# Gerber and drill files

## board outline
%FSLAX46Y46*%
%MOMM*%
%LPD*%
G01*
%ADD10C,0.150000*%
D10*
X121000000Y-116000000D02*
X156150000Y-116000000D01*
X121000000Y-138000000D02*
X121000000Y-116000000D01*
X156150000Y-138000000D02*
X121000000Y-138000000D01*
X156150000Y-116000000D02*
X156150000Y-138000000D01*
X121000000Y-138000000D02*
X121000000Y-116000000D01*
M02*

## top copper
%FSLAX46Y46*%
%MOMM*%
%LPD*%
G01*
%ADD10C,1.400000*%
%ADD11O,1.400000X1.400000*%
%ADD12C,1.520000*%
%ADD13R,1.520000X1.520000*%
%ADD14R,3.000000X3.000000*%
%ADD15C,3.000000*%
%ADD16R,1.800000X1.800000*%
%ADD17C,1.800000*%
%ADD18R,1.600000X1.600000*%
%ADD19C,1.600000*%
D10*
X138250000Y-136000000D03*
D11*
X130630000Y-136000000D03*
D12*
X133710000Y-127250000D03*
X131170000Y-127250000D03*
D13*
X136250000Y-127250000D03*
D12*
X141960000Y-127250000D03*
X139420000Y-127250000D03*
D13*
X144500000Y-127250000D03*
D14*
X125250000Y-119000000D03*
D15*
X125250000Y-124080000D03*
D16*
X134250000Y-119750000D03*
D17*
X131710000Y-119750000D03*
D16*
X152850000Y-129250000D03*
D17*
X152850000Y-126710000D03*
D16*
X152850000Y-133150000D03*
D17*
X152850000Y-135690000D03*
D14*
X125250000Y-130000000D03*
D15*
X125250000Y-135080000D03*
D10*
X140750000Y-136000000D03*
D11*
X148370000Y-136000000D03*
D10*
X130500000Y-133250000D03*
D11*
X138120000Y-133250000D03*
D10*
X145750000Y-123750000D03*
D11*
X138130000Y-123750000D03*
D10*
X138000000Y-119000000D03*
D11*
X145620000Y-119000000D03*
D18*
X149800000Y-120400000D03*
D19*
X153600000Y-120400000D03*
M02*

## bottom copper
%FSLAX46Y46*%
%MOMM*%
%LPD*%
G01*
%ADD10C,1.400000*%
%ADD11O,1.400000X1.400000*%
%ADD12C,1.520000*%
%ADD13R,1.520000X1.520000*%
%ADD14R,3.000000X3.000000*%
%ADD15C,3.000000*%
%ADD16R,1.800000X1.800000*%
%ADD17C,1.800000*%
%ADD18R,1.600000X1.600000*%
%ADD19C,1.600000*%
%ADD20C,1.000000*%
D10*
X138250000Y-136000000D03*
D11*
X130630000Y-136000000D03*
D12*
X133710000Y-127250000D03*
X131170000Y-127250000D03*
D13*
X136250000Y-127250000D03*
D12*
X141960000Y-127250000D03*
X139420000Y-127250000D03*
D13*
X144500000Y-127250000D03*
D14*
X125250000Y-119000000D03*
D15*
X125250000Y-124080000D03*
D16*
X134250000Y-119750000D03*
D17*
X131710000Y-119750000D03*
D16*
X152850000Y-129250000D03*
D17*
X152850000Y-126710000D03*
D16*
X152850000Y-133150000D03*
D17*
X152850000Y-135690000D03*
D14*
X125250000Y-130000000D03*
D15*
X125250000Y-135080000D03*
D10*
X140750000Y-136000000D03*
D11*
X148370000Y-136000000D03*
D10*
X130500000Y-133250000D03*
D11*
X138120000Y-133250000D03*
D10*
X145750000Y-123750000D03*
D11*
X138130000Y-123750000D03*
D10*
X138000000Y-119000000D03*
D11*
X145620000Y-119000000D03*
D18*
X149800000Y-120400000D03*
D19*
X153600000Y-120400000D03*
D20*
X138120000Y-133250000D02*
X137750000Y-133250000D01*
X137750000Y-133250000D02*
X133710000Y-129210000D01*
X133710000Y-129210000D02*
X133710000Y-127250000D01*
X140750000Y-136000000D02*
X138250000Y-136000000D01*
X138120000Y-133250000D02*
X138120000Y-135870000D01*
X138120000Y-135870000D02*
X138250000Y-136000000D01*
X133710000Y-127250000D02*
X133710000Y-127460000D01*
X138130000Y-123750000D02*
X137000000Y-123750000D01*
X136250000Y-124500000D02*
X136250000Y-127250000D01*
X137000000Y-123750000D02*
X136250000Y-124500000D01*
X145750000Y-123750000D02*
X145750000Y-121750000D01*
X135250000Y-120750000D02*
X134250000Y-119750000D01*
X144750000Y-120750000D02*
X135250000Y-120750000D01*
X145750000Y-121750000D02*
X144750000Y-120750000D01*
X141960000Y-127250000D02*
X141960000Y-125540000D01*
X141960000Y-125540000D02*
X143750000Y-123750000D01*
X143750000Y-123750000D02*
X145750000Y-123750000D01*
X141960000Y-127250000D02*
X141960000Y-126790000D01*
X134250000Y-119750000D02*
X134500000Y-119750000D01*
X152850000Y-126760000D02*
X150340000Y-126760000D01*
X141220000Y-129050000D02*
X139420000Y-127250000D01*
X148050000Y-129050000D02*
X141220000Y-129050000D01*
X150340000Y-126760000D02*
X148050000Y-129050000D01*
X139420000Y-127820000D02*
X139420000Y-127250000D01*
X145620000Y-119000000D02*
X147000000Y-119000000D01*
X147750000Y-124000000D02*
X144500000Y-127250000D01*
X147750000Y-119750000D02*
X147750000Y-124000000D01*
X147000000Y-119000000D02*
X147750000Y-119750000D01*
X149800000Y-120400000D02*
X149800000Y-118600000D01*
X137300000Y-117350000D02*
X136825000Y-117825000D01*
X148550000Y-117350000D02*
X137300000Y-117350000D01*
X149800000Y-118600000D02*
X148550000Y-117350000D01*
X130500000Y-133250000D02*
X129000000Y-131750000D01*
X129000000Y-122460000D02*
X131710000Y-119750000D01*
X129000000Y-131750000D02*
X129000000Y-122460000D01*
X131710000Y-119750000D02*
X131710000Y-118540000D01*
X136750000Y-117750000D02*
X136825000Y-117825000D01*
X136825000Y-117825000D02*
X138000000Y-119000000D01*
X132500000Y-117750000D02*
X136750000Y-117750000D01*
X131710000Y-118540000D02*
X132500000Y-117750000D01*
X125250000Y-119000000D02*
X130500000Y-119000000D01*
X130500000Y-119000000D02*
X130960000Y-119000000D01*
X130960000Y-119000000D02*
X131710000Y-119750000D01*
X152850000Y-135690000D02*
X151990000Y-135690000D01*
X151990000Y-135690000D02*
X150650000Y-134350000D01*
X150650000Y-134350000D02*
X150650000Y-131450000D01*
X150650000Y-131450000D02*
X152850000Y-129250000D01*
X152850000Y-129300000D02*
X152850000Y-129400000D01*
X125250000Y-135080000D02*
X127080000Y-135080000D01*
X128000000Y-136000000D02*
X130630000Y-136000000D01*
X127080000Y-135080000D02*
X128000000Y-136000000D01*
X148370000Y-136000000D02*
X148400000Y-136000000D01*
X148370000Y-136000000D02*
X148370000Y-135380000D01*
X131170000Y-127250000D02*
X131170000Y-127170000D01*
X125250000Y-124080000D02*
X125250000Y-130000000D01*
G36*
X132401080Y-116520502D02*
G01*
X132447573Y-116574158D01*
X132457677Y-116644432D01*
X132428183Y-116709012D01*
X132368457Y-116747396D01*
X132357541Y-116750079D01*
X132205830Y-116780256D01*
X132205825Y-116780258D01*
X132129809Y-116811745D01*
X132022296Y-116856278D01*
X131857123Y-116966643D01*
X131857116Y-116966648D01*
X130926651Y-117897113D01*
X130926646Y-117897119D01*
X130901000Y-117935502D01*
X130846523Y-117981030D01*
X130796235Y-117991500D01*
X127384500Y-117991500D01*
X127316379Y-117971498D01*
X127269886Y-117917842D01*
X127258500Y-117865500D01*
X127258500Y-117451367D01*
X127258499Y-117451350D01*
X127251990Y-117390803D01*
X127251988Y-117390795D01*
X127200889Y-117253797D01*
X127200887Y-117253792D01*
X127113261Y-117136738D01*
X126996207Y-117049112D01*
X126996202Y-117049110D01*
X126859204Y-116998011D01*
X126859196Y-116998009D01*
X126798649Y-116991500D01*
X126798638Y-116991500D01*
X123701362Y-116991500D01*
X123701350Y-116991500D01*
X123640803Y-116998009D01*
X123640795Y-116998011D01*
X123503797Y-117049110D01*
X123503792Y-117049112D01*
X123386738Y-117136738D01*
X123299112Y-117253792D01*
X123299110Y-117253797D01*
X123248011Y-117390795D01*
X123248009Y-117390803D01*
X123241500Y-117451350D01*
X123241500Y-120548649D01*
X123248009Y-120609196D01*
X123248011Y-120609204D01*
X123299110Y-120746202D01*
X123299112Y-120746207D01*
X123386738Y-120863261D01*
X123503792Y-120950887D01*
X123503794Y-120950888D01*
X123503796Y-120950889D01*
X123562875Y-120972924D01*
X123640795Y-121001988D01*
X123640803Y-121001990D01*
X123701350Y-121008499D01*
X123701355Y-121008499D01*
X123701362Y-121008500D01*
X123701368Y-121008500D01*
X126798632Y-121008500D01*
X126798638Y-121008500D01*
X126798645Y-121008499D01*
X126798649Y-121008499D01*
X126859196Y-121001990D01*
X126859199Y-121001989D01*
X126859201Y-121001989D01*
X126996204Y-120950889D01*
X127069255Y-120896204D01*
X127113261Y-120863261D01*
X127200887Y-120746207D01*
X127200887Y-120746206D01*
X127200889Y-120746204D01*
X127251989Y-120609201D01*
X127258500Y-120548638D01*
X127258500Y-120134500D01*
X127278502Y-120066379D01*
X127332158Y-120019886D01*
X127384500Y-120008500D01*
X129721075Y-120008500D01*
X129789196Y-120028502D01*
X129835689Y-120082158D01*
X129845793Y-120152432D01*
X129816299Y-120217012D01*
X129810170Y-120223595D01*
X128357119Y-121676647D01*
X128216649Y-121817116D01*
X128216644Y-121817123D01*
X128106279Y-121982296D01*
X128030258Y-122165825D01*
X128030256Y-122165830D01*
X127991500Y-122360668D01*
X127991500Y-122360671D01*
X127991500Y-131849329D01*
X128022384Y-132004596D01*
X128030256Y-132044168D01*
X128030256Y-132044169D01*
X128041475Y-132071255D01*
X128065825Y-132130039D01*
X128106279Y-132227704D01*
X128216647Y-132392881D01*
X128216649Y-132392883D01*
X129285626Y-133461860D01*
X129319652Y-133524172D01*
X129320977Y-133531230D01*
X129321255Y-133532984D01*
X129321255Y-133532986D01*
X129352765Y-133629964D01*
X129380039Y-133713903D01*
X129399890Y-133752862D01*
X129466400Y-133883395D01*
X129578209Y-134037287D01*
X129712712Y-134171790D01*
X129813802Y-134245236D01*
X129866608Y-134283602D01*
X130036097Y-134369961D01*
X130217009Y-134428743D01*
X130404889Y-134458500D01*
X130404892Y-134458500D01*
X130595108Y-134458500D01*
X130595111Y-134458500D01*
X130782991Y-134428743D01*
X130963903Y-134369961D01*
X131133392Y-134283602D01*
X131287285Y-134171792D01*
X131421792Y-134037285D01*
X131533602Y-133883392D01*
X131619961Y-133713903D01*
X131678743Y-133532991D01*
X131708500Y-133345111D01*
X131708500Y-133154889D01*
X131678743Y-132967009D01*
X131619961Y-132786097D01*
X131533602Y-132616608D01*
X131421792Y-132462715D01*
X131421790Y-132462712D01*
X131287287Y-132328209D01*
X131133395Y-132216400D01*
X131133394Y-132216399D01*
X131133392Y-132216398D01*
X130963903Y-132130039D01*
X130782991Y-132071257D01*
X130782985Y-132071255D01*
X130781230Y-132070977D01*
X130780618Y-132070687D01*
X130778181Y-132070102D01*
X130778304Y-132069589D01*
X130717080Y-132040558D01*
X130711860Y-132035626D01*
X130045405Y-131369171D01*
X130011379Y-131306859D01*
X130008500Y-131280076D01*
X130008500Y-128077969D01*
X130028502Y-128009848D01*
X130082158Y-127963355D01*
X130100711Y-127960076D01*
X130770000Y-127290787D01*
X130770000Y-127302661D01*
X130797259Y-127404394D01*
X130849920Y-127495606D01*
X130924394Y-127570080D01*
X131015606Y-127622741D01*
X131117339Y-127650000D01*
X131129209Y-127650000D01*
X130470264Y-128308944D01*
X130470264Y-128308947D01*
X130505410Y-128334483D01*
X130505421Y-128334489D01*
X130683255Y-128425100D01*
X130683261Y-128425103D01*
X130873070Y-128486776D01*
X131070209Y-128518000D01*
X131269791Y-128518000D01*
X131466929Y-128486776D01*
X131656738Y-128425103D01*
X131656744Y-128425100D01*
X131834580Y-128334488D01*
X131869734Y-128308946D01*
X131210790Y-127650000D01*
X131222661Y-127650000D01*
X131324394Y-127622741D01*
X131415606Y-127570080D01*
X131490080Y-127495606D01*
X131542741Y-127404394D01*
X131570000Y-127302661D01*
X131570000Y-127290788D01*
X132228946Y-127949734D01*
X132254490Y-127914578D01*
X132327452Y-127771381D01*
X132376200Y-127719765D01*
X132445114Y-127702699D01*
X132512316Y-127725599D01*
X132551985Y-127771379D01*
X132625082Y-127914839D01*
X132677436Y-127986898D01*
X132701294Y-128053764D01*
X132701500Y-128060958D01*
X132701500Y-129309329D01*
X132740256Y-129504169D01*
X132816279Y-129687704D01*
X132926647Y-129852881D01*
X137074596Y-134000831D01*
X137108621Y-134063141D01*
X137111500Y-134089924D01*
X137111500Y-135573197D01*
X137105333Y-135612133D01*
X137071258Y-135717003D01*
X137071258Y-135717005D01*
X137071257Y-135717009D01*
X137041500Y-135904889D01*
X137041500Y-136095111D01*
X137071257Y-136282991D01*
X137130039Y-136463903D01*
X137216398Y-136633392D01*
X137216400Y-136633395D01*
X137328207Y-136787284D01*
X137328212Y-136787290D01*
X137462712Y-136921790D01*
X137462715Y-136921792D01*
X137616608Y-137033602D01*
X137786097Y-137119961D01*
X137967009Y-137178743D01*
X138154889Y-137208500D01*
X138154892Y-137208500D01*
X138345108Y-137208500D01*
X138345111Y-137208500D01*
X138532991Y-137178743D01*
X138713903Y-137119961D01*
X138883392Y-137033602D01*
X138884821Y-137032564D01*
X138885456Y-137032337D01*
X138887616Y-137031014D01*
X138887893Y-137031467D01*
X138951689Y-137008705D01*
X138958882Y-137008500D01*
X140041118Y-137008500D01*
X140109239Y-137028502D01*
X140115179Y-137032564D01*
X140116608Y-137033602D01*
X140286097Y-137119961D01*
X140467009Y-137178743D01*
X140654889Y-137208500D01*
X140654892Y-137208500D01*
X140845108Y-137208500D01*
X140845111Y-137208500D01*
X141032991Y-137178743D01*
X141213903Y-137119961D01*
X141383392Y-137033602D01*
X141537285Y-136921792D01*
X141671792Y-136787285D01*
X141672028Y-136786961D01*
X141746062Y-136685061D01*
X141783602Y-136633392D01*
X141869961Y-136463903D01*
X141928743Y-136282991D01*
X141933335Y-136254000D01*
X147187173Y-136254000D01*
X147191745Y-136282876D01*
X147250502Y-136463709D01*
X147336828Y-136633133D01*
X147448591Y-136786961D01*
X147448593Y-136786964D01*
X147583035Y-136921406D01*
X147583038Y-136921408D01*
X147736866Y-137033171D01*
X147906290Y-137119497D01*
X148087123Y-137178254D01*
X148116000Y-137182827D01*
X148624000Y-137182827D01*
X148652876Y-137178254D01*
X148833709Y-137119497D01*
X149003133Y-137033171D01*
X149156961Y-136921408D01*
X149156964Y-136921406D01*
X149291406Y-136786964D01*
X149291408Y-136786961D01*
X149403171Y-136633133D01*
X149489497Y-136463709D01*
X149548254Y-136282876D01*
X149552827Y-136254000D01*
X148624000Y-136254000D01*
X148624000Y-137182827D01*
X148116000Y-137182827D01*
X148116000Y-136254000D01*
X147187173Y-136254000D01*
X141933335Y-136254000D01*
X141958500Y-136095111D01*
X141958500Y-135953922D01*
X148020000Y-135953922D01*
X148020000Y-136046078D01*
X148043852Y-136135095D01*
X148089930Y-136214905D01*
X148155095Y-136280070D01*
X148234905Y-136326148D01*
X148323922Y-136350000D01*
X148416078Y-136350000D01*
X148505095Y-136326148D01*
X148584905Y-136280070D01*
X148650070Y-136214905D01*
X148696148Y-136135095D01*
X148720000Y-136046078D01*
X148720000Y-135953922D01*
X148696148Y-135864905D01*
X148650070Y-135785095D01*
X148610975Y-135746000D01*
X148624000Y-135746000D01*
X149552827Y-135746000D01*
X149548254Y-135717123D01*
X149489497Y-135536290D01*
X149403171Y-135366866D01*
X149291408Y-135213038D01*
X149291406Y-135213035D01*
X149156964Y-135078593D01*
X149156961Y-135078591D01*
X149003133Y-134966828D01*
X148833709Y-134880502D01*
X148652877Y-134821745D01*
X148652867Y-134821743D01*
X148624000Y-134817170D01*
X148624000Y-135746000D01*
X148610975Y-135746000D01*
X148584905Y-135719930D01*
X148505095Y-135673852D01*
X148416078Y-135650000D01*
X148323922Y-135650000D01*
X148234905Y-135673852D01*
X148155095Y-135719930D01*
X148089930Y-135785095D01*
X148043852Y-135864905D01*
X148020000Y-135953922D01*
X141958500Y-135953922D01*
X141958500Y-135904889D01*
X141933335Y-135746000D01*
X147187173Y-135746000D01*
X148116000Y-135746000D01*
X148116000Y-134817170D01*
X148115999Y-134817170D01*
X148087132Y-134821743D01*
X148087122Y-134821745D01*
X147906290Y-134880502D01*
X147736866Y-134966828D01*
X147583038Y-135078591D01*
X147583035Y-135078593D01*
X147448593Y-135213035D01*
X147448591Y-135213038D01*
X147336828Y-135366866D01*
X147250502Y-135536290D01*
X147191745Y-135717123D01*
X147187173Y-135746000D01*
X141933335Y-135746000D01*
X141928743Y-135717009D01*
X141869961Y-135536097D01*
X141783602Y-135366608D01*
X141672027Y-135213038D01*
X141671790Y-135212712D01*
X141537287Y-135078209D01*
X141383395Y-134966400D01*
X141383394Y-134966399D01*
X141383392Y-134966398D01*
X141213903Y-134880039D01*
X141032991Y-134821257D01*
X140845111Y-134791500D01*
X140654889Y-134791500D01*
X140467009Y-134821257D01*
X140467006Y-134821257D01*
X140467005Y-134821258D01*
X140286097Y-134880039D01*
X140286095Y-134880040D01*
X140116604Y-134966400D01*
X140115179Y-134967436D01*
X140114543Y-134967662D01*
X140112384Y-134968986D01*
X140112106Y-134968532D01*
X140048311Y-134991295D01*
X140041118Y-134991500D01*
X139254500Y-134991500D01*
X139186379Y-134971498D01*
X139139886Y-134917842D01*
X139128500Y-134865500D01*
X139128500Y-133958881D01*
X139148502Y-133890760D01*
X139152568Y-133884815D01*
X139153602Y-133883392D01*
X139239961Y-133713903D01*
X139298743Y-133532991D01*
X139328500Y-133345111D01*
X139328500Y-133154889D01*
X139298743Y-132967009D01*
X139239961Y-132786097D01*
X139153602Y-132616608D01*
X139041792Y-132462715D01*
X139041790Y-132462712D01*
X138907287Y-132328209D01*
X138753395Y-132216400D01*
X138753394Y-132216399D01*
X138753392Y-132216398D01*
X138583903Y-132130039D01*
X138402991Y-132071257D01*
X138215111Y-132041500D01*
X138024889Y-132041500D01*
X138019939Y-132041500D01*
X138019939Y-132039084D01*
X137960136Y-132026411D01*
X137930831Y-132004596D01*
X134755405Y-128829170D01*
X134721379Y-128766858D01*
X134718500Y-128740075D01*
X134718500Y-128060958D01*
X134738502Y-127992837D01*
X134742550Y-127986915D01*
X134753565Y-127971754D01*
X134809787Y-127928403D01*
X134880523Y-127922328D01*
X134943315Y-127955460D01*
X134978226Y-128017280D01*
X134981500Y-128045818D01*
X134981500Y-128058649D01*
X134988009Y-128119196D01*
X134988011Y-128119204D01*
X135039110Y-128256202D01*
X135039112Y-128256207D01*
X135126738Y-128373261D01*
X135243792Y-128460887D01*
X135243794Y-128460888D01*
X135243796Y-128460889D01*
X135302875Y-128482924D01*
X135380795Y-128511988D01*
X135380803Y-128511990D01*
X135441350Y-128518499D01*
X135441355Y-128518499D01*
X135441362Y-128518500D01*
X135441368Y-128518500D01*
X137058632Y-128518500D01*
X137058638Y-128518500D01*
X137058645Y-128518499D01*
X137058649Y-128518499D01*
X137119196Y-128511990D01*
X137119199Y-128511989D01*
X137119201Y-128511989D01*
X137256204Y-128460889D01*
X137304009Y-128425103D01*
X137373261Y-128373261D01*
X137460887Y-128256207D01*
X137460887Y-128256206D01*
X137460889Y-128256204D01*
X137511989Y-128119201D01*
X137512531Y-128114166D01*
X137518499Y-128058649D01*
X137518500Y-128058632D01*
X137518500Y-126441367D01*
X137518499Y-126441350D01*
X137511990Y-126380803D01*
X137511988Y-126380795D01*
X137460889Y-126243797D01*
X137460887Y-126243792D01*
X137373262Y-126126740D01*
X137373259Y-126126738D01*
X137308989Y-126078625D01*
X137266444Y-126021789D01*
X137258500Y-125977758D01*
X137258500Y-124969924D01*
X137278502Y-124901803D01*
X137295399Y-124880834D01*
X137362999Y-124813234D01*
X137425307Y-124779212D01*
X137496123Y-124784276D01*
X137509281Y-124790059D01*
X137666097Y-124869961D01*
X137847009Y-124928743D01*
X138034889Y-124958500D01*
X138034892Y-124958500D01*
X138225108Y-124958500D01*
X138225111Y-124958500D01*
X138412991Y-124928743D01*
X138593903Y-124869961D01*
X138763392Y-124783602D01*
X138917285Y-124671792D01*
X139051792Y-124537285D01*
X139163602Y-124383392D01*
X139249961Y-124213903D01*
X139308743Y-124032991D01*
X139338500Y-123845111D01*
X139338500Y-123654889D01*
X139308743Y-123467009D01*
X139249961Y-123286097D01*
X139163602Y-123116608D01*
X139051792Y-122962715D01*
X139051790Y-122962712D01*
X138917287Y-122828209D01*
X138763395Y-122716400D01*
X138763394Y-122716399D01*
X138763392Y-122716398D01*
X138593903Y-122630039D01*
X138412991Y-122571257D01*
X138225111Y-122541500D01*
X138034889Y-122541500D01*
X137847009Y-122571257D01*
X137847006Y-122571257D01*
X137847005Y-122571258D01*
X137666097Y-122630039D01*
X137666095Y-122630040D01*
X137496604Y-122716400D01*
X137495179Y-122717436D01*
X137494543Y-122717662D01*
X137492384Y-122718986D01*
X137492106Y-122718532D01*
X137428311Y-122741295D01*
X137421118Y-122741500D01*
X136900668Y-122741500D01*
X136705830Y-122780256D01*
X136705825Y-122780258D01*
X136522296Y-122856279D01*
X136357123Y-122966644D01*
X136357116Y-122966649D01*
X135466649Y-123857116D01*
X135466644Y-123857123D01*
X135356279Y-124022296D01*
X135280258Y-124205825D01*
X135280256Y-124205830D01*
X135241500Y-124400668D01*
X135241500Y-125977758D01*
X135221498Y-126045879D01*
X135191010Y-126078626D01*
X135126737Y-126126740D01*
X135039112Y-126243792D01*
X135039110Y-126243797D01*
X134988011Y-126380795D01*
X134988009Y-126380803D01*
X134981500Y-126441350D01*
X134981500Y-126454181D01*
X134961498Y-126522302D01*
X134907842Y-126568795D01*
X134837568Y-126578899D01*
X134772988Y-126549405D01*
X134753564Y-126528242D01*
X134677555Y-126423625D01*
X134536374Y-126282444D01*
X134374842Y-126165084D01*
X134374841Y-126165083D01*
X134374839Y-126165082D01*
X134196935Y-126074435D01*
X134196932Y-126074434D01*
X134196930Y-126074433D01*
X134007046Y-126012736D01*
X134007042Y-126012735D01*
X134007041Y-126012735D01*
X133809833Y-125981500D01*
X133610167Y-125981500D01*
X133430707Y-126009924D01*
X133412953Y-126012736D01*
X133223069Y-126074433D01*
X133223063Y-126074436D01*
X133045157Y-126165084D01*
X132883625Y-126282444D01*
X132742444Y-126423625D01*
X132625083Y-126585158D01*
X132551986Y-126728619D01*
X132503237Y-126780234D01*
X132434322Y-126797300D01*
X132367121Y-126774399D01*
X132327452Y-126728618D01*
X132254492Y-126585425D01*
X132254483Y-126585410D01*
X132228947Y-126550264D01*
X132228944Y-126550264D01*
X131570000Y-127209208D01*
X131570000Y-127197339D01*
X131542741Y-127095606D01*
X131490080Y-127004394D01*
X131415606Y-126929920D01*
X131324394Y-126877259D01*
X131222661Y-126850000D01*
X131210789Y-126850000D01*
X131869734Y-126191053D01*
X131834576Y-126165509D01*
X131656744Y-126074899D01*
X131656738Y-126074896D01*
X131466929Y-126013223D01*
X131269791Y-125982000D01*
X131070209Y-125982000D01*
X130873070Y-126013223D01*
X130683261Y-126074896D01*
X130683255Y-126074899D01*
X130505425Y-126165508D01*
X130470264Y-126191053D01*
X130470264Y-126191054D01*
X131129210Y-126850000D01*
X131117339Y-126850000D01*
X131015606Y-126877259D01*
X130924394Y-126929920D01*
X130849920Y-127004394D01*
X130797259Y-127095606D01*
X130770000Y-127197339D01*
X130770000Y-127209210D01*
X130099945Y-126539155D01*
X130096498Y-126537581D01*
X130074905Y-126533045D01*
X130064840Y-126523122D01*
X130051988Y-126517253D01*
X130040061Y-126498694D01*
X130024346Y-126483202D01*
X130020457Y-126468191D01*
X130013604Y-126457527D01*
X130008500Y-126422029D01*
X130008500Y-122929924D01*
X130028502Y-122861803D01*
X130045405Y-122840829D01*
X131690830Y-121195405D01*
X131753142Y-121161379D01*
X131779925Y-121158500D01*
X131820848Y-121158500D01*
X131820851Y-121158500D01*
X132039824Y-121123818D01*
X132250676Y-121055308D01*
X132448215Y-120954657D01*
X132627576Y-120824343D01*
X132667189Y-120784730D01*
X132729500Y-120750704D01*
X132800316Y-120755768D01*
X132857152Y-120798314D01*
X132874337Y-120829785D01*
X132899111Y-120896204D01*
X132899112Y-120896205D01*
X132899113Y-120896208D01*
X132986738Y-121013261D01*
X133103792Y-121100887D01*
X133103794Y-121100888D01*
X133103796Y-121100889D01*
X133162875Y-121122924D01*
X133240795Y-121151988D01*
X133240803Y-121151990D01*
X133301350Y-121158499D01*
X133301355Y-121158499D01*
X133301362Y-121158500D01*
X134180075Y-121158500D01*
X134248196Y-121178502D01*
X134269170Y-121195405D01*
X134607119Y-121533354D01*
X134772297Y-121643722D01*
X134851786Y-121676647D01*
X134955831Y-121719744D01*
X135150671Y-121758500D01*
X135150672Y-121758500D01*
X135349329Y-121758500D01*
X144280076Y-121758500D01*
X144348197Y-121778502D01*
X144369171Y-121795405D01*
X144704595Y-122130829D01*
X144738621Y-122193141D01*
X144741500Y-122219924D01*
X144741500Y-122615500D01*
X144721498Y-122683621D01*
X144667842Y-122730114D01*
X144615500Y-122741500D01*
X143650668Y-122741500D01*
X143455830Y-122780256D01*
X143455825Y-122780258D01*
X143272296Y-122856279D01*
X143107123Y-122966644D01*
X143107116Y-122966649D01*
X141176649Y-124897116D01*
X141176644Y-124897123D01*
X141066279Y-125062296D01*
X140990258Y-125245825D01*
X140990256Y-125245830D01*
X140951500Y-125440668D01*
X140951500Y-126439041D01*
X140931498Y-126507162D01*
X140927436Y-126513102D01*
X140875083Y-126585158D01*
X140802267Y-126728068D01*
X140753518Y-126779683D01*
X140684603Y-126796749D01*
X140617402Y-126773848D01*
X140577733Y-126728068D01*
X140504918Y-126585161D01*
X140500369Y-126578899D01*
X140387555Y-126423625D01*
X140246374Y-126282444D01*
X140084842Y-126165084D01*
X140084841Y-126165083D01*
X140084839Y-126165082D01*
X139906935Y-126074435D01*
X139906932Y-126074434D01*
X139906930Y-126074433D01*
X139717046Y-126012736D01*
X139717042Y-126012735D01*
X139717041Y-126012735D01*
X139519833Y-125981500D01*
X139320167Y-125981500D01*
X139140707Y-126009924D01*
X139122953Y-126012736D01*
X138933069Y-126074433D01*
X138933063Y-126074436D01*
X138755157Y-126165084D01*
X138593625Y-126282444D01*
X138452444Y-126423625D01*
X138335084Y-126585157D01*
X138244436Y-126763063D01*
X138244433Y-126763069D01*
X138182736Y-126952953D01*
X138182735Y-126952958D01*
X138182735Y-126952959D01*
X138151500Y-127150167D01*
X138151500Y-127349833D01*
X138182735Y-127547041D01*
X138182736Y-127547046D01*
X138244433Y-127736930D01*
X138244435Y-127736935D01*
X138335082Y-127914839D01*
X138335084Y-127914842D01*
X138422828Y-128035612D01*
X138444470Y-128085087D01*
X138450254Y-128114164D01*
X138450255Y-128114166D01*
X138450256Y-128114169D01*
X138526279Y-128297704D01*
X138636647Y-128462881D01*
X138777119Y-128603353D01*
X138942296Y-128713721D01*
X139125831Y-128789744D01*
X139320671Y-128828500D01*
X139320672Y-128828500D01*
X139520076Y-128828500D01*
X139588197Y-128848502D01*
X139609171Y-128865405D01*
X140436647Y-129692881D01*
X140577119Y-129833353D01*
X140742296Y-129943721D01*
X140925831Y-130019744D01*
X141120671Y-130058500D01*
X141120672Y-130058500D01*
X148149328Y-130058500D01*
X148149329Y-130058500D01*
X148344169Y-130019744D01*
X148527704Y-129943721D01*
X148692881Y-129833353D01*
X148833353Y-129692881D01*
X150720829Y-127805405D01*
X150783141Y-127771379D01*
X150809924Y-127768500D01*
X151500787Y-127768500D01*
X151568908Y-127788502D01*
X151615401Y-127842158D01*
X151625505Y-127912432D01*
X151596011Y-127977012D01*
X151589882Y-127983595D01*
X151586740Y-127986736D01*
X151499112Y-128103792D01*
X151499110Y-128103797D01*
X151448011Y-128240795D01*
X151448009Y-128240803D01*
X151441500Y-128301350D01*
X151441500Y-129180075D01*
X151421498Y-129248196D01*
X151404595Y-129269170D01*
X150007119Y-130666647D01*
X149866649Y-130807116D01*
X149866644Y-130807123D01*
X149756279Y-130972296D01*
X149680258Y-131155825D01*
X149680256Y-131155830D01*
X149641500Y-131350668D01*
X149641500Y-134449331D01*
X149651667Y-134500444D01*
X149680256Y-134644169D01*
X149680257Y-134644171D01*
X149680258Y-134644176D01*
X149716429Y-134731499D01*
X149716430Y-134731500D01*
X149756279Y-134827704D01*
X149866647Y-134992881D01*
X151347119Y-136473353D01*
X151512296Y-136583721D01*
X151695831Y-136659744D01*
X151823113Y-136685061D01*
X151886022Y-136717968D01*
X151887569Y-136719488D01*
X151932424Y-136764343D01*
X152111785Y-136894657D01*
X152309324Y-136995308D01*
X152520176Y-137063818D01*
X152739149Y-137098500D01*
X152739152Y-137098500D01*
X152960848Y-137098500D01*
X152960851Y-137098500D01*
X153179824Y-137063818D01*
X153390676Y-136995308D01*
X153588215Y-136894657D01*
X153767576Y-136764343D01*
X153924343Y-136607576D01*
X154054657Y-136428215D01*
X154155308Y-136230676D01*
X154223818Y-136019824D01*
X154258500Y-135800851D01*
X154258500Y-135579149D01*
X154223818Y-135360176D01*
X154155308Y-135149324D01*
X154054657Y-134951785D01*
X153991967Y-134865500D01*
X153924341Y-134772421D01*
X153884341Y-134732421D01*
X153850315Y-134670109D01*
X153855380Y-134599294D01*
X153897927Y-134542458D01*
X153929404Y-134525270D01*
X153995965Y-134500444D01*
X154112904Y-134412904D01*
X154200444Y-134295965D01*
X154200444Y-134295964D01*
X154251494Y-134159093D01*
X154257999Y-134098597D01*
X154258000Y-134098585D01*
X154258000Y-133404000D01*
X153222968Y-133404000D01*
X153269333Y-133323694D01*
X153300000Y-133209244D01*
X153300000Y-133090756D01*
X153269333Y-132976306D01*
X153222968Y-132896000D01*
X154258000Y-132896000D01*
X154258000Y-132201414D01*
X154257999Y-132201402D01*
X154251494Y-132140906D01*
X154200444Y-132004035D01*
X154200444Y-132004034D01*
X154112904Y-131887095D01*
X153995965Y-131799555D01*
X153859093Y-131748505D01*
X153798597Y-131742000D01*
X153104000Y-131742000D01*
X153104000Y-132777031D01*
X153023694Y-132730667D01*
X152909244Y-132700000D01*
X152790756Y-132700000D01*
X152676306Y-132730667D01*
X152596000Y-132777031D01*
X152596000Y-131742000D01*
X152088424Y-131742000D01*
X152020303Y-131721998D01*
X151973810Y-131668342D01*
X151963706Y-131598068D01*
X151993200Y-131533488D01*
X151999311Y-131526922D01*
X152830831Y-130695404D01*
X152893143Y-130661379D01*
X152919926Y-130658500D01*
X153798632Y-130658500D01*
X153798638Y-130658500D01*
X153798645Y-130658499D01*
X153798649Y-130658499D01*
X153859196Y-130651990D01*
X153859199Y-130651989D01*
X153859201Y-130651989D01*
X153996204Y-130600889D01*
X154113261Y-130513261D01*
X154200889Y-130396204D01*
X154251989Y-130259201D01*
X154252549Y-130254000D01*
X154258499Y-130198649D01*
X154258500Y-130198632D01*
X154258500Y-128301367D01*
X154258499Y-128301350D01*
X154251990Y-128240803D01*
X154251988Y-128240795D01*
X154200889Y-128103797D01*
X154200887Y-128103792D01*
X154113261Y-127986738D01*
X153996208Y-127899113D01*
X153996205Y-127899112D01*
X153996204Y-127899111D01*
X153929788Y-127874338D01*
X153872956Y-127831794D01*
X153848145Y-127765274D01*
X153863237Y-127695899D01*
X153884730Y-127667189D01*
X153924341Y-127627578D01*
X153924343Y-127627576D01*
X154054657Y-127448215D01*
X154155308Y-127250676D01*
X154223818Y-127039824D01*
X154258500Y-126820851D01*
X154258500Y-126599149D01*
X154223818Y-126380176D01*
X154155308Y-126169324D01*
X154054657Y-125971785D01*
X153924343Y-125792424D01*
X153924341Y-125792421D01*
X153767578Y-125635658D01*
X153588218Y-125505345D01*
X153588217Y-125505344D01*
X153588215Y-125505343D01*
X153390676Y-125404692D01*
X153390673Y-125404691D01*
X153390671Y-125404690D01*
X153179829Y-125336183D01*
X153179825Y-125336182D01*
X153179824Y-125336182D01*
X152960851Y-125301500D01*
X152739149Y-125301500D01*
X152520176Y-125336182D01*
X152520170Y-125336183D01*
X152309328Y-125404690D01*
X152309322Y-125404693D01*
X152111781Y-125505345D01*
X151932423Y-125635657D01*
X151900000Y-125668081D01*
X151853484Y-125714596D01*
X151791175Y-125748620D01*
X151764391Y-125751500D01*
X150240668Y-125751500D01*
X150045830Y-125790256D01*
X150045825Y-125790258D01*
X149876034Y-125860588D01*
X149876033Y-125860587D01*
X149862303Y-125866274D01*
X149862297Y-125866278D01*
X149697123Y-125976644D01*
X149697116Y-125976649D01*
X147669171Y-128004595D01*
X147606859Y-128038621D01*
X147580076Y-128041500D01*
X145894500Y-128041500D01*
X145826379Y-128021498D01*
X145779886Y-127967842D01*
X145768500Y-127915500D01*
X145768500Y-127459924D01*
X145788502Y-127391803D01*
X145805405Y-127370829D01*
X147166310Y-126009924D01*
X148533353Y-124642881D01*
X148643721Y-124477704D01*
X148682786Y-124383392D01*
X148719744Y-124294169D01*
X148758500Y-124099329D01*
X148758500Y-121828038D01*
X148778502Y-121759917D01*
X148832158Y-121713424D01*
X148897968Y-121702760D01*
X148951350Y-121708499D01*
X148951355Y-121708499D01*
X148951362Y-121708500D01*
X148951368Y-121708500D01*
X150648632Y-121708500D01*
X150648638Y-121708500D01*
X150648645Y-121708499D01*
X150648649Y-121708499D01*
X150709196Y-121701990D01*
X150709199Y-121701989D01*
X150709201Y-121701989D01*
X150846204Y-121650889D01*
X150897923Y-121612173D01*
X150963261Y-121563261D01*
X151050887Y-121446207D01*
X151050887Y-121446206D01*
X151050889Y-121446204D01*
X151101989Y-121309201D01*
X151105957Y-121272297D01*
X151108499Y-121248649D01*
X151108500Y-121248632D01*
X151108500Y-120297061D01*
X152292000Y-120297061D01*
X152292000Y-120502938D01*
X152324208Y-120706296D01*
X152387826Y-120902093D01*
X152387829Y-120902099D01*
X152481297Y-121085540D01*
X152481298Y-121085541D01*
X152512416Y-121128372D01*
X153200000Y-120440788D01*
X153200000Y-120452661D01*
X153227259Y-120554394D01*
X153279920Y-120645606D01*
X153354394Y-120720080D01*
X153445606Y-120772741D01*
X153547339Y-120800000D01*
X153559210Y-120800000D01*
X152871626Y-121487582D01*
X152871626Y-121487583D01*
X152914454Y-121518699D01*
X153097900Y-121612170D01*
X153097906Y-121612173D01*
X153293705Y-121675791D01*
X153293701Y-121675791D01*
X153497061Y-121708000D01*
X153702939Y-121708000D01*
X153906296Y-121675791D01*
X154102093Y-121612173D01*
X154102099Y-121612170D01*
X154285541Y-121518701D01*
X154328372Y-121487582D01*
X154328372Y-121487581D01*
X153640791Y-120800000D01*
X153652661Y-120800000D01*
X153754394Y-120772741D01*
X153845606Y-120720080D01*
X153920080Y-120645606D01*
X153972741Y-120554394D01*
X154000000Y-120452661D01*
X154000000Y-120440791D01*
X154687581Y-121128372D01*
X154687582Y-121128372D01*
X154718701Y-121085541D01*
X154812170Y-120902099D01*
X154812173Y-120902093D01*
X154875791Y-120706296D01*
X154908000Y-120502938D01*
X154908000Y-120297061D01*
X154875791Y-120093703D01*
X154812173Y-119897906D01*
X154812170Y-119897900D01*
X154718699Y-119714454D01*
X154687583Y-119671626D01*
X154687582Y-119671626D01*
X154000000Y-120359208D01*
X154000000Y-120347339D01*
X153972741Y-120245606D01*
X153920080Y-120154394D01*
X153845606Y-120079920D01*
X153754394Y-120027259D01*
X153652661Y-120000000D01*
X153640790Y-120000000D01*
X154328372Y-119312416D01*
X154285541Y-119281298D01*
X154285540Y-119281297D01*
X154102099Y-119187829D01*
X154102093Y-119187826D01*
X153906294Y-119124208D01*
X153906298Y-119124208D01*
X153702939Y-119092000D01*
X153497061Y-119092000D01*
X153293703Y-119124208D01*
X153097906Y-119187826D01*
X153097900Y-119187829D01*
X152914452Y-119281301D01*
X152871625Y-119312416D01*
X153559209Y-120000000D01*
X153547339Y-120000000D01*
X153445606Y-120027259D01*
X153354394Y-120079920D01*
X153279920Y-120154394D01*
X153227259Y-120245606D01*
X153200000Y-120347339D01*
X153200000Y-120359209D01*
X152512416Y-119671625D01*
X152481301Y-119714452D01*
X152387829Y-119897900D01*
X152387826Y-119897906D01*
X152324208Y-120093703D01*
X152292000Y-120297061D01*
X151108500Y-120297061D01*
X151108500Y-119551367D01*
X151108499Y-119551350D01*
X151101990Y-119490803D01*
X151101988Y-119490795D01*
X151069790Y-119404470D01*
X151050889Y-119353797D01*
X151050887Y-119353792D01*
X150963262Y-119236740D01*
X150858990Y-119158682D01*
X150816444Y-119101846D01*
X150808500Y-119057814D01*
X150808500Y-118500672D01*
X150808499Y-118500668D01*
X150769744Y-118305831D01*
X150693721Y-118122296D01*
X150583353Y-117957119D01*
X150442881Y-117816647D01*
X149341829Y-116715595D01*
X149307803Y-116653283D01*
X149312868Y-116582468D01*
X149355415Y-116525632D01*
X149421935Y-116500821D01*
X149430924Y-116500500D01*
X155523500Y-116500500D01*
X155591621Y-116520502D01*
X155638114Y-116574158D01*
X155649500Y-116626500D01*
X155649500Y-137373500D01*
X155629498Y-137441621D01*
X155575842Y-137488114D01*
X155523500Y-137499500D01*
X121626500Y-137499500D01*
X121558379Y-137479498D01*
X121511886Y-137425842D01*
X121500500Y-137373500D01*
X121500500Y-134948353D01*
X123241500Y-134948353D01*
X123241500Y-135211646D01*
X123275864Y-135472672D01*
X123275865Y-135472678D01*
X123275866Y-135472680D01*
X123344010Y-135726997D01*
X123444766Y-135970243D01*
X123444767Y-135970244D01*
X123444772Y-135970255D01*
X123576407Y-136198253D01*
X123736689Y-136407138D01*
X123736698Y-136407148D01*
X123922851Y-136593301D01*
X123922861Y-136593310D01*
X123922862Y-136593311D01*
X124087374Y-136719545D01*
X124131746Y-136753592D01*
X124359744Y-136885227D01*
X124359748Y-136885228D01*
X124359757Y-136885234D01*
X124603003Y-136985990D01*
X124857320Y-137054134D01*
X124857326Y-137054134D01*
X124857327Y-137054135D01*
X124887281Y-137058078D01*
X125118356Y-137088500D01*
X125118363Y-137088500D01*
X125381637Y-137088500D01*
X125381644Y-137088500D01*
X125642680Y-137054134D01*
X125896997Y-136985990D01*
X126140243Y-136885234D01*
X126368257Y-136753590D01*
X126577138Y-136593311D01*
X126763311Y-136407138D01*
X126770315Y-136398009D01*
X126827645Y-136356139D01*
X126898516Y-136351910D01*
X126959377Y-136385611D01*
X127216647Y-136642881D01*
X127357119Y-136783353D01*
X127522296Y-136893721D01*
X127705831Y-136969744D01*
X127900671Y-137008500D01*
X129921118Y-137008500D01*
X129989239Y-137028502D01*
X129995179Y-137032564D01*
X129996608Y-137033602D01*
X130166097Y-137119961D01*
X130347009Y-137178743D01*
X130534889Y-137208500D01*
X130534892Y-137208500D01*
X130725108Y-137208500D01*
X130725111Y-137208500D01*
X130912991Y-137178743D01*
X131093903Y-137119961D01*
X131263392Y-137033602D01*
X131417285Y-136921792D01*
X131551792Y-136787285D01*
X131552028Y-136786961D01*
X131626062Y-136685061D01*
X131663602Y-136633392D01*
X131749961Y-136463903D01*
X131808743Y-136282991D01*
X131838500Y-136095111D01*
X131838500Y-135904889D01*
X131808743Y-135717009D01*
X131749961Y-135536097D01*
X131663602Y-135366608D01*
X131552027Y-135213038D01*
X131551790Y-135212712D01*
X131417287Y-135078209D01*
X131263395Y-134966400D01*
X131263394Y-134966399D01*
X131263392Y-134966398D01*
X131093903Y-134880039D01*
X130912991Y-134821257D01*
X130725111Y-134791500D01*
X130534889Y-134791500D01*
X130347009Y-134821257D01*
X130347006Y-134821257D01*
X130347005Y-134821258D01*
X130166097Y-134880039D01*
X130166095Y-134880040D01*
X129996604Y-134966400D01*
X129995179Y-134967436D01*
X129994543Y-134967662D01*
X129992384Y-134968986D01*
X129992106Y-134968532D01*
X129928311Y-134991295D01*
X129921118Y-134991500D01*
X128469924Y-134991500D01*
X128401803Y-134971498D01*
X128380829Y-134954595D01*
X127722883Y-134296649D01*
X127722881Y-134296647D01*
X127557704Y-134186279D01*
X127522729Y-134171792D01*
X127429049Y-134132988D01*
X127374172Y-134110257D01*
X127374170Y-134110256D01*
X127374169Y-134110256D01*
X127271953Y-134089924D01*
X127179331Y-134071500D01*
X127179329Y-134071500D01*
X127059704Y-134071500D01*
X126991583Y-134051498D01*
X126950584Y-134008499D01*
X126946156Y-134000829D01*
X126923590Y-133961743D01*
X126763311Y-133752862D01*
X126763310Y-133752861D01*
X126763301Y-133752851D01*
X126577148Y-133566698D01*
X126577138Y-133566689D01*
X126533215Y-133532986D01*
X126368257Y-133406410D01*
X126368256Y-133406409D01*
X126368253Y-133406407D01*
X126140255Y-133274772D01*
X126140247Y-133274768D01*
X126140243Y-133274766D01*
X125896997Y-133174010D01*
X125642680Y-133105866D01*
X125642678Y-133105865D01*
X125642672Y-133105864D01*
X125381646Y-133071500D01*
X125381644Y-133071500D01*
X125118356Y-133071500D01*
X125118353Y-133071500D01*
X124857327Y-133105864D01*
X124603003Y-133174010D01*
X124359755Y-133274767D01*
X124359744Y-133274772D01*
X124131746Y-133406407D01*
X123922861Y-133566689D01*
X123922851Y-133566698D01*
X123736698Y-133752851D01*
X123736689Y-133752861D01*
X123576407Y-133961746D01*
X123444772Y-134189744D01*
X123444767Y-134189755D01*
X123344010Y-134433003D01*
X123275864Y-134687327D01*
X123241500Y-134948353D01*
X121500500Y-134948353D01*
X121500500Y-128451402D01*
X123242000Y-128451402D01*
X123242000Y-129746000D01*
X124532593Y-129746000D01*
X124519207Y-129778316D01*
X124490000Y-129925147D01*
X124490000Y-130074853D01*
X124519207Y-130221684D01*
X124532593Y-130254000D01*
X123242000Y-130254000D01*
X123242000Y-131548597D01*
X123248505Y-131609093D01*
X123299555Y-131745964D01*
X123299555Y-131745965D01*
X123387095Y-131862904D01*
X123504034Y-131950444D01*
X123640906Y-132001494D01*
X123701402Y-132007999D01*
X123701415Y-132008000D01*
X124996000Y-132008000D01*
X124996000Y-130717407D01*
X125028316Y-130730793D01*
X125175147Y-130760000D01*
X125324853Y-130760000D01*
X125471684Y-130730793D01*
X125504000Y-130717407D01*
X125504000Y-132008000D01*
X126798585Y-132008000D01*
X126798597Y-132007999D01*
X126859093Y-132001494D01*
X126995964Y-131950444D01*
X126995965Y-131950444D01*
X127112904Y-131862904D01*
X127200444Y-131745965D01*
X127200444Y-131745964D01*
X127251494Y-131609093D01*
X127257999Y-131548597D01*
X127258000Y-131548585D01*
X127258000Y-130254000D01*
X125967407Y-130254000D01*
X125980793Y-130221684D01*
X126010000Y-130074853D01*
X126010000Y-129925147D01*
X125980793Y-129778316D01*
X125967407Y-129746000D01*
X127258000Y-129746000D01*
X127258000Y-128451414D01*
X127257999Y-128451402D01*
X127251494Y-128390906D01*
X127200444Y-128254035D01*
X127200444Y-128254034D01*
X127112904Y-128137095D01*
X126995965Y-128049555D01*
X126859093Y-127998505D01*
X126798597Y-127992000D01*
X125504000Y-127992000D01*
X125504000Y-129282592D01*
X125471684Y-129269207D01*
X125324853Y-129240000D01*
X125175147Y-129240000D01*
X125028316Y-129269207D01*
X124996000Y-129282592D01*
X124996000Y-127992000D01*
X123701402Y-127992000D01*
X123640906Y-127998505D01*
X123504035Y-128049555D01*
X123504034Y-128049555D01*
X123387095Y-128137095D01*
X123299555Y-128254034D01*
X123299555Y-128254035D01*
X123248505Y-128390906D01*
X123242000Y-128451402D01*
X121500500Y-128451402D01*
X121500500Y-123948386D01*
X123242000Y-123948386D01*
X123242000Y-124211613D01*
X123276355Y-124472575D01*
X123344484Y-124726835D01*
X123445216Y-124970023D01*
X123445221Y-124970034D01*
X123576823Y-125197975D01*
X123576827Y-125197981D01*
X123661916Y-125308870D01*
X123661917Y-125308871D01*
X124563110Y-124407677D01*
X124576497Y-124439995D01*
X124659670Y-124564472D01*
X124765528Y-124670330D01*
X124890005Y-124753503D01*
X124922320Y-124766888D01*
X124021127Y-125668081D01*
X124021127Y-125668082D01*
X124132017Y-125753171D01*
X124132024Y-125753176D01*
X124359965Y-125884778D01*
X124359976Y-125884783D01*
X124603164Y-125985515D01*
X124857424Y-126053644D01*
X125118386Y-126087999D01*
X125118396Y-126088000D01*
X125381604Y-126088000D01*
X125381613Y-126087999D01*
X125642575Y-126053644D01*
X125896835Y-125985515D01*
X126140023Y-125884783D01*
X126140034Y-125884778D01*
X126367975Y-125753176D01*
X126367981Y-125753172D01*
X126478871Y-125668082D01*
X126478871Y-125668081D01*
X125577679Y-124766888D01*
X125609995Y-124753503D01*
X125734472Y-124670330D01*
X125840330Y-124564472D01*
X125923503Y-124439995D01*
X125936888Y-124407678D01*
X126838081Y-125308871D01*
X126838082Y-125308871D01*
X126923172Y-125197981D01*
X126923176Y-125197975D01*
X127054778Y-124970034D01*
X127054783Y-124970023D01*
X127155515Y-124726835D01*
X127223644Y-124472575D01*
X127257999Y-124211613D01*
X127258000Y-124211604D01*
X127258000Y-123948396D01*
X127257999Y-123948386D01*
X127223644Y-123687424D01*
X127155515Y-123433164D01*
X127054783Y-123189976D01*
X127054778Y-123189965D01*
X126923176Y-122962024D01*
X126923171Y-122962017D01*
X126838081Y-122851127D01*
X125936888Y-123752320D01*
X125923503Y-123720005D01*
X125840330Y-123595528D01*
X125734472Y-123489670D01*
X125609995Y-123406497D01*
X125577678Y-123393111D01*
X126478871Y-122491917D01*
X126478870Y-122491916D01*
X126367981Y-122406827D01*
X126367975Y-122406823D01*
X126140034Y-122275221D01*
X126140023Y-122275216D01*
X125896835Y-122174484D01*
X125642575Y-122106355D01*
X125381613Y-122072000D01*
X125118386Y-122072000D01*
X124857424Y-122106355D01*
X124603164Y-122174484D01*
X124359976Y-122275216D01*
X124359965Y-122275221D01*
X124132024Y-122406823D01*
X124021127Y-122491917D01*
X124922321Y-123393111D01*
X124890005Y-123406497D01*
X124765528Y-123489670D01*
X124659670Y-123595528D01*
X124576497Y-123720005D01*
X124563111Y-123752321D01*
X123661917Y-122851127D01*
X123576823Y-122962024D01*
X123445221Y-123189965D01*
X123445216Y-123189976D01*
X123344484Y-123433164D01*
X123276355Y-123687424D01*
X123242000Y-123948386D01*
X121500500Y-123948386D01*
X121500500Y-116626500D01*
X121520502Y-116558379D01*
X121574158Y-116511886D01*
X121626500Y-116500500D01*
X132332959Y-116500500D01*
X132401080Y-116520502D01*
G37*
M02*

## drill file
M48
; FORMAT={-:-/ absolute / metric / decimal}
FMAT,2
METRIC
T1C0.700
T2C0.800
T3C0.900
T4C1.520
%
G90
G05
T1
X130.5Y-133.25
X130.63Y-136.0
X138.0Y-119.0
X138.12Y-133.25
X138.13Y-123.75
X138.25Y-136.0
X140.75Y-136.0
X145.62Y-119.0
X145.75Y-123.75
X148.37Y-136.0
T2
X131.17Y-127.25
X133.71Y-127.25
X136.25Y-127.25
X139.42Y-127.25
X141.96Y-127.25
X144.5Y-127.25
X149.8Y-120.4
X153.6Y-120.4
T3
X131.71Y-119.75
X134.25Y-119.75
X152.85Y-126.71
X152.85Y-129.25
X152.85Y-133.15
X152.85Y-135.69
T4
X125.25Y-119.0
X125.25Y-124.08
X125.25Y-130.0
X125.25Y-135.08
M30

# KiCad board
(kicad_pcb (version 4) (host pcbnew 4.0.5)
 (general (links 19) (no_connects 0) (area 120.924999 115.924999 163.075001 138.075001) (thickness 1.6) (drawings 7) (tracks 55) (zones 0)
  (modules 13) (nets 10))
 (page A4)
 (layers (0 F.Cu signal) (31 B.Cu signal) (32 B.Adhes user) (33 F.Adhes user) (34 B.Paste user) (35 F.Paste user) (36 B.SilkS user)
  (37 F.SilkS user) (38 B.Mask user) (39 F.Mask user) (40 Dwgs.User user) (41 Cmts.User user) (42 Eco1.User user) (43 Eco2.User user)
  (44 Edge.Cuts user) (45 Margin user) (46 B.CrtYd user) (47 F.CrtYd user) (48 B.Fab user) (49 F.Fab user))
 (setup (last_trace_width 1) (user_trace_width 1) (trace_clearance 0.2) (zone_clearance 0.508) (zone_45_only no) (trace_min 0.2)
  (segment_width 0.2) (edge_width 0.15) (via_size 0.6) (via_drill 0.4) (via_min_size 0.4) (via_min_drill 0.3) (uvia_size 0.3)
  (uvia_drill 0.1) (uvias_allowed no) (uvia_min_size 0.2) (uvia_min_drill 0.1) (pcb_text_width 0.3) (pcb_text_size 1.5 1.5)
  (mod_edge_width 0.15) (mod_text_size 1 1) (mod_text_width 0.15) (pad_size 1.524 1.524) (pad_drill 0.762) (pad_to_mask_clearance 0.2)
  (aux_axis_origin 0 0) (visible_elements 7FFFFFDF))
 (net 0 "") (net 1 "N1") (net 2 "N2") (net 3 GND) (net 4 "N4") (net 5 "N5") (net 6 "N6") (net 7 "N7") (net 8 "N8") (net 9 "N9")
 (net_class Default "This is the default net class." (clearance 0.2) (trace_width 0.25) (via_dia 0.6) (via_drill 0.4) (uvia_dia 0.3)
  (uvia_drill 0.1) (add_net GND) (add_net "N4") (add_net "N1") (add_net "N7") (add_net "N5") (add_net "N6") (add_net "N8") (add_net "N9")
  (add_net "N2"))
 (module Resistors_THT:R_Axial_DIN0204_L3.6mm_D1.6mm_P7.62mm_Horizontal (layer F.Cu) (at 138.25 136 180)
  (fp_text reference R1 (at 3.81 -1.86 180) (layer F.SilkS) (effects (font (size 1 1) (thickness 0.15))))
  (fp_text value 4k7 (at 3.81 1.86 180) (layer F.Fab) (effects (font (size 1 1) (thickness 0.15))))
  (pad 1 thru_hole circle (at 0 0 180) (size 1.4 1.4) (drill 0.7) (layers *.Cu *.Mask) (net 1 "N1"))
  (pad 2 thru_hole oval (at 7.62 0 180) (size 1.4 1.4) (drill 0.7) (layers *.Cu *.Mask) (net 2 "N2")))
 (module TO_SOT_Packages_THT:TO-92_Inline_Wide (layer F.Cu) (at 136.25 127.25 180)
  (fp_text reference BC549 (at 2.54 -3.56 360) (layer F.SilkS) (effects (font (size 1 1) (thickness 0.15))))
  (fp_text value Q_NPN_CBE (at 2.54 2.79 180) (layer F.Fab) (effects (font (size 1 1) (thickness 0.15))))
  (pad 2 thru_hole circle (at 2.54 0 270) (size 1.52 1.52) (drill 0.8) (layers *.Cu *.Mask) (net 1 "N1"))
  (pad 3 thru_hole circle (at 5.08 0 270) (size 1.52 1.52) (drill 0.8) (layers *.Cu *.Mask) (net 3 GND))
  (pad 1 thru_hole rect (at 0 0 270) (size 1.52 1.52) (drill 0.8) (layers *.Cu *.Mask) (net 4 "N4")))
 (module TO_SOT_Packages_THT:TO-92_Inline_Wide (layer F.Cu) (at 144.5 127.25 180)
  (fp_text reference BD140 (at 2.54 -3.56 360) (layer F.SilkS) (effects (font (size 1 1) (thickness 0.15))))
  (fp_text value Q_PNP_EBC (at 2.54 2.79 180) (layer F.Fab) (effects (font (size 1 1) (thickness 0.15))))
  (pad 2 thru_hole circle (at 2.54 0 270) (size 1.52 1.52) (drill 0.8) (layers *.Cu *.Mask) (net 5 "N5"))
  (pad 3 thru_hole circle (at 5.08 0 270) (size 1.52 1.52) (drill 0.8) (layers *.Cu *.Mask) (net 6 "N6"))
  (pad 1 thru_hole rect (at 0 0 270) (size 1.52 1.52) (drill 0.8) (layers *.Cu *.Mask) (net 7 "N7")))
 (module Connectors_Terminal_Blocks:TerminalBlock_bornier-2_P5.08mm (layer F.Cu) (at 125.25 119 270)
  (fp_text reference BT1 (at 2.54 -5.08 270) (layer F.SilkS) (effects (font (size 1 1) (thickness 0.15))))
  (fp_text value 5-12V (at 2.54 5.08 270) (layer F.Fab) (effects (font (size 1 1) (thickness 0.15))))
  (pad 1 thru_hole rect (at 0 0 270) (size 3 3) (drill 1.52) (layers *.Cu *.Mask) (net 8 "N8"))
  (pad 2 thru_hole circle (at 5.08 0 270) (size 3 3) (drill 1.52) (layers *.Cu *.Mask) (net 3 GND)))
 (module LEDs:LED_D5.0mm (layer F.Cu) (at 134.25 119.75 180)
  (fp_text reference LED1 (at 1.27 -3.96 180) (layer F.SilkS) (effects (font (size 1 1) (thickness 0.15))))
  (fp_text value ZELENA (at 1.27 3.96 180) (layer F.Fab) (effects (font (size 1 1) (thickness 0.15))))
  (pad 1 thru_hole rect (at 0 0 180) (size 1.8 1.8) (drill 0.9) (layers *.Cu *.Mask) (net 5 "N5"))
  (pad 2 thru_hole circle (at 2.54 0 180) (size 1.8 1.8) (drill 0.9) (layers *.Cu *.Mask) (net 8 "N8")))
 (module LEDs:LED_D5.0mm (layer F.Cu) (at 152.85 129.25 90)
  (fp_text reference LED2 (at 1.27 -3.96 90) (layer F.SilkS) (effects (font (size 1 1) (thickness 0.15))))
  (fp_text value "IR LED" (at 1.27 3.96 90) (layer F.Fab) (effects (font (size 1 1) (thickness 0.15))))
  (pad 1 thru_hole rect (at 0 0 90) (size 1.8 1.8) (drill 0.9) (layers *.Cu *.Mask) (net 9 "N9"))
  (pad 2 thru_hole circle (at 2.54 0 90) (size 1.8 1.8) (drill 0.9) (layers *.Cu *.Mask) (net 6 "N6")))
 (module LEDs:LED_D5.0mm (layer F.Cu) (at 152.85 133.15 270)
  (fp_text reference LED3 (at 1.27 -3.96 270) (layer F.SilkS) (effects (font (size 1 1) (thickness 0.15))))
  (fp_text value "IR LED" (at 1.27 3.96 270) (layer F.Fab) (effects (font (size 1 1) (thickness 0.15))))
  (pad 1 thru_hole rect (at 0 0 270) (size 1.8 1.8) (drill 0.9) (layers *.Cu *.Mask) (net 3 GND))
  (pad 2 thru_hole circle (at 2.54 0 270) (size 1.8 1.8) (drill 0.9) (layers *.Cu *.Mask) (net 9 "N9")))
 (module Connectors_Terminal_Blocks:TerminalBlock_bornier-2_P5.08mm (layer F.Cu) (at 125.25 130 270)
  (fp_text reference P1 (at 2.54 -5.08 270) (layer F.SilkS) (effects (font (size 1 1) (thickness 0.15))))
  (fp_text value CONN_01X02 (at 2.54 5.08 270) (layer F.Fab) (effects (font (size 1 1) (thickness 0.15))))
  (pad 1 thru_hole rect (at 0 0 270) (size 3 3) (drill 1.52) (layers *.Cu *.Mask) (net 3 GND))
  (pad 2 thru_hole circle (at 5.08 0 270) (size 3 3) (drill 1.52) (layers *.Cu *.Mask) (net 2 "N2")))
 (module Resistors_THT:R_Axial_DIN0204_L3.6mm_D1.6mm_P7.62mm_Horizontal (layer F.Cu) (at 140.75 136)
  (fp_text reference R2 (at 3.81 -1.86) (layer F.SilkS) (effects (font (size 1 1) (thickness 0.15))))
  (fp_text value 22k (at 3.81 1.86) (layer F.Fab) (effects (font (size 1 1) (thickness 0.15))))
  (pad 1 thru_hole circle (at 0 0) (size 1.4 1.4) (drill 0.7) (layers *.Cu *.Mask) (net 1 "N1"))
  (pad 2 thru_hole oval (at 7.62 0) (size 1.4 1.4) (drill 0.7) (layers *.Cu *.Mask) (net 3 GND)))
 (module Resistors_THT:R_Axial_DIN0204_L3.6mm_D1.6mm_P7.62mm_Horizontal (layer F.Cu) (at 130.5 133.25)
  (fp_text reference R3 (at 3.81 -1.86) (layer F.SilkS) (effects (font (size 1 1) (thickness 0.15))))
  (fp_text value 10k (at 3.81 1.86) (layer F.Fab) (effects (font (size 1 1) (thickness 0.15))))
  (pad 1 thru_hole circle (at 0 0) (size 1.4 1.4) (drill 0.7) (layers *.Cu *.Mask) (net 8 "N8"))
  (pad 2 thru_hole oval (at 7.62 0) (size 1.4 1.4) (drill 0.7) (layers *.Cu *.Mask) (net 1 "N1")))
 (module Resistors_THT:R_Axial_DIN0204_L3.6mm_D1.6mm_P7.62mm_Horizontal (layer F.Cu) (at 145.75 123.75 180)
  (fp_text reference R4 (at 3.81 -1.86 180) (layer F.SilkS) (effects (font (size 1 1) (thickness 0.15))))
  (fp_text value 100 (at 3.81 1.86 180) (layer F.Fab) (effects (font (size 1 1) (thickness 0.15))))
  (pad 1 thru_hole circle (at 0 0 180) (size 1.4 1.4) (drill 0.7) (layers *.Cu *.Mask) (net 5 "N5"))
  (pad 2 thru_hole oval (at 7.62 0 180) (size 1.4 1.4) (drill 0.7) (layers *.Cu *.Mask) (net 4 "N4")))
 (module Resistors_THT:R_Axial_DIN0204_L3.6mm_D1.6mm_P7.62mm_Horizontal (layer F.Cu) (at 138 119)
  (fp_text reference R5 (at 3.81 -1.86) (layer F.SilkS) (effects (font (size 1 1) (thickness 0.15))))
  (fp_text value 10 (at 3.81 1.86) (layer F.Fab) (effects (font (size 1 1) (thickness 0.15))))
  (pad 1 thru_hole circle (at 0 0) (size 1.4 1.4) (drill 0.7) (layers *.Cu *.Mask) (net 8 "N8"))
  (pad 2 thru_hole oval (at 7.62 0) (size 1.4 1.4) (drill 0.7) (layers *.Cu *.Mask) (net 7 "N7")))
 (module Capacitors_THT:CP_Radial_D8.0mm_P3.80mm (layer F.Cu) (at 149.8 120.4)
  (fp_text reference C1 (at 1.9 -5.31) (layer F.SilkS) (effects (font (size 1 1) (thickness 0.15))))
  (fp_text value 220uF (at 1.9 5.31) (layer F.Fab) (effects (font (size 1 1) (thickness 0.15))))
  (pad 1 thru_hole rect (at 0 0) (size 1.6 1.6) (drill 0.8) (layers *.Cu *.Mask) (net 8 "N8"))
  (pad 2 thru_hole circle (at 3.8 0) (size 1.6 1.6) (drill 0.8) (layers *.Cu *.Mask) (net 3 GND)))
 (gr_line (start 121 116) (end 156.15 116) (angle 90) (layer Edge.Cuts) (width 0.15))
 (gr_line (start 121 138) (end 121 116) (angle 90) (layer Edge.Cuts) (width 0.15))
 (gr_line (start 156.15 138) (end 121 138) (angle 90) (layer Edge.Cuts) (width 0.15))
 (gr_line (start 156.15 116) (end 156.15 138) (angle 90) (layer Edge.Cuts) (width 0.15))
 (gr_line (start 121 138) (end 121 116) (angle 90) (layer Edge.Cuts) (width 0.15))
 (segment (start 138.12 133.25) (end 137.75 133.25) (width 1) (layer B.Cu) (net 1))
 (segment (start 137.75 133.25) (end 133.71 129.21) (width 1) (layer B.Cu) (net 1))
 (segment (start 133.71 129.21) (end 133.71 127.25) (width 1) (layer B.Cu) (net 1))
 (segment (start 140.75 136) (end 138.25 136) (width 1) (layer B.Cu) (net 1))
 (segment (start 138.12 133.25) (end 138.12 135.87) (width 1) (layer B.Cu) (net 1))
 (segment (start 138.12 135.87) (end 138.25 136) (width 1) (layer B.Cu) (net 1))
 (segment (start 133.71 127.25) (end 133.71 127.46) (width 1) (layer B.Cu) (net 1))
 (segment (start 138.13 123.75) (end 137 123.75) (width 1) (layer B.Cu) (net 4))
 (segment (start 136.25 124.5) (end 136.25 127.25) (width 1) (layer B.Cu) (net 4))
 (segment (start 137 123.75) (end 136.25 124.5) (width 1) (layer B.Cu) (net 4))
 (segment (start 145.75 123.75) (end 145.75 121.75) (width 1) (layer B.Cu) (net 5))
 (segment (start 135.25 120.75) (end 134.25 119.75) (width 1) (layer B.Cu) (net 5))
 (segment (start 144.75 120.75) (end 135.25 120.75) (width 1) (layer B.Cu) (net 5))
 (segment (start 145.75 121.75) (end 144.75 120.75) (width 1) (layer B.Cu) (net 5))
 (segment (start 141.96 127.25) (end 141.96 125.54) (width 1) (layer B.Cu) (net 5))
 (segment (start 141.96 125.54) (end 143.75 123.75) (width 1) (layer B.Cu) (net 5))
 (segment (start 143.75 123.75) (end 145.75 123.75) (width 1) (layer B.Cu) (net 5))
 (segment (start 141.96 127.25) (end 141.96 126.79) (width 1) (layer B.Cu) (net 5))
 (segment (start 134.25 119.75) (end 134.5 119.75) (width 1) (layer B.Cu) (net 5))
 (segment (start 152.85 126.76) (end 150.34 126.76) (width 1) (layer B.Cu) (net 6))
 (segment (start 141.22 129.05) (end 139.42 127.25) (width 1) (layer B.Cu) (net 6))
 (segment (start 148.05 129.05) (end 141.22 129.05) (width 1) (layer B.Cu) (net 6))
 (segment (start 150.34 126.76) (end 148.05 129.05) (width 1) (layer B.Cu) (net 6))
 (segment (start 139.42 127.82) (end 139.42 127.25) (width 1) (layer B.Cu) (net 6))
 (segment (start 145.62 119) (end 147 119) (width 1) (layer B.Cu) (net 7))
 (segment (start 147.75 124) (end 144.5 127.25) (width 1) (layer B.Cu) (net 7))
 (segment (start 147.75 119.75) (end 147.75 124) (width 1) (layer B.Cu) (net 7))
 (segment (start 147 119) (end 147.75 119.75) (width 1) (layer B.Cu) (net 7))
 (segment (start 149.8 120.4) (end 149.8 118.6) (width 1) (layer B.Cu) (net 8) (status 400000))
 (segment (start 137.3 117.35) (end 136.825 117.825) (width 1) (layer B.Cu) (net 8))
 (segment (start 148.55 117.35) (end 137.3 117.35) (width 1) (layer B.Cu) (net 8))
 (segment (start 149.8 118.6) (end 148.55 117.35) (width 1) (layer B.Cu) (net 8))
 (segment (start 130.5 133.25) (end 129 131.75) (width 1) (layer B.Cu) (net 8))
 (segment (start 129 122.46) (end 131.71 119.75) (width 1) (layer B.Cu) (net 8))
 (segment (start 129 131.75) (end 129 122.46) (width 1) (layer B.Cu) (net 8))
 (segment (start 131.71 119.75) (end 131.71 118.54) (width 1) (layer B.Cu) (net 8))
 (segment (start 136.75 117.75) (end 136.825 117.825) (width 1) (layer B.Cu) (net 8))
 (segment (start 136.825 117.825) (end 138 119) (width 1) (layer B.Cu) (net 8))
 (segment (start 132.5 117.75) (end 136.75 117.75) (width 1) (layer B.Cu) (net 8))
 (segment (start 131.71 118.54) (end 132.5 117.75) (width 1) (layer B.Cu) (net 8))
 (segment (start 125.25 119) (end 130.5 119) (width 1) (layer B.Cu) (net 8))
 (segment (start 130.5 119) (end 130.96 119) (width 1) (layer B.Cu) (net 8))
 (segment (start 130.96 119) (end 131.71 119.75) (width 1) (layer B.Cu) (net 8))
 (segment (start 152.85 135.69) (end 151.99 135.69) (width 1) (layer B.Cu) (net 9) (status C00000))
 (segment (start 151.99 135.69) (end 150.65 134.35) (width 1) (layer B.Cu) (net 9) (status 400000))
 (segment (start 150.65 134.35) (end 150.65 131.45) (width 1) (layer B.Cu) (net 9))
 (segment (start 150.65 131.45) (end 152.85 129.25) (width 1) (layer B.Cu) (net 9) (status 800000))
 (segment (start 152.85 129.3) (end 152.85 129.4) (width 1) (layer B.Cu) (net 9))
 (segment (start 125.25 135.08) (end 127.08 135.08) (width 1) (layer B.Cu) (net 2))
 (segment (start 128 136) (end 130.63 136) (width 1) (layer B.Cu) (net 2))
 (segment (start 127.08 135.08) (end 128 136) (width 1) (layer B.Cu) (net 2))
 (segment (start 148.37 136) (end 148.4 136) (width 1) (layer B.Cu) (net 3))
 (segment (start 148.37 136) (end 148.37 135.38) (width 1) (layer B.Cu) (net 3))
 (segment (start 131.17 127.25) (end 131.17 127.17) (width 1) (layer B.Cu) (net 3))
 (segment (start 125.25 124.08) (end 125.25 130) (width 1) (layer B.Cu) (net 3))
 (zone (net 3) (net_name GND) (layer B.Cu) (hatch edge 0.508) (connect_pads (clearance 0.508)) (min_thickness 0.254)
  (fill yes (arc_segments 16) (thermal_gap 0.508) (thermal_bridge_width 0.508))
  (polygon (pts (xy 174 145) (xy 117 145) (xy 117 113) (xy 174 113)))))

